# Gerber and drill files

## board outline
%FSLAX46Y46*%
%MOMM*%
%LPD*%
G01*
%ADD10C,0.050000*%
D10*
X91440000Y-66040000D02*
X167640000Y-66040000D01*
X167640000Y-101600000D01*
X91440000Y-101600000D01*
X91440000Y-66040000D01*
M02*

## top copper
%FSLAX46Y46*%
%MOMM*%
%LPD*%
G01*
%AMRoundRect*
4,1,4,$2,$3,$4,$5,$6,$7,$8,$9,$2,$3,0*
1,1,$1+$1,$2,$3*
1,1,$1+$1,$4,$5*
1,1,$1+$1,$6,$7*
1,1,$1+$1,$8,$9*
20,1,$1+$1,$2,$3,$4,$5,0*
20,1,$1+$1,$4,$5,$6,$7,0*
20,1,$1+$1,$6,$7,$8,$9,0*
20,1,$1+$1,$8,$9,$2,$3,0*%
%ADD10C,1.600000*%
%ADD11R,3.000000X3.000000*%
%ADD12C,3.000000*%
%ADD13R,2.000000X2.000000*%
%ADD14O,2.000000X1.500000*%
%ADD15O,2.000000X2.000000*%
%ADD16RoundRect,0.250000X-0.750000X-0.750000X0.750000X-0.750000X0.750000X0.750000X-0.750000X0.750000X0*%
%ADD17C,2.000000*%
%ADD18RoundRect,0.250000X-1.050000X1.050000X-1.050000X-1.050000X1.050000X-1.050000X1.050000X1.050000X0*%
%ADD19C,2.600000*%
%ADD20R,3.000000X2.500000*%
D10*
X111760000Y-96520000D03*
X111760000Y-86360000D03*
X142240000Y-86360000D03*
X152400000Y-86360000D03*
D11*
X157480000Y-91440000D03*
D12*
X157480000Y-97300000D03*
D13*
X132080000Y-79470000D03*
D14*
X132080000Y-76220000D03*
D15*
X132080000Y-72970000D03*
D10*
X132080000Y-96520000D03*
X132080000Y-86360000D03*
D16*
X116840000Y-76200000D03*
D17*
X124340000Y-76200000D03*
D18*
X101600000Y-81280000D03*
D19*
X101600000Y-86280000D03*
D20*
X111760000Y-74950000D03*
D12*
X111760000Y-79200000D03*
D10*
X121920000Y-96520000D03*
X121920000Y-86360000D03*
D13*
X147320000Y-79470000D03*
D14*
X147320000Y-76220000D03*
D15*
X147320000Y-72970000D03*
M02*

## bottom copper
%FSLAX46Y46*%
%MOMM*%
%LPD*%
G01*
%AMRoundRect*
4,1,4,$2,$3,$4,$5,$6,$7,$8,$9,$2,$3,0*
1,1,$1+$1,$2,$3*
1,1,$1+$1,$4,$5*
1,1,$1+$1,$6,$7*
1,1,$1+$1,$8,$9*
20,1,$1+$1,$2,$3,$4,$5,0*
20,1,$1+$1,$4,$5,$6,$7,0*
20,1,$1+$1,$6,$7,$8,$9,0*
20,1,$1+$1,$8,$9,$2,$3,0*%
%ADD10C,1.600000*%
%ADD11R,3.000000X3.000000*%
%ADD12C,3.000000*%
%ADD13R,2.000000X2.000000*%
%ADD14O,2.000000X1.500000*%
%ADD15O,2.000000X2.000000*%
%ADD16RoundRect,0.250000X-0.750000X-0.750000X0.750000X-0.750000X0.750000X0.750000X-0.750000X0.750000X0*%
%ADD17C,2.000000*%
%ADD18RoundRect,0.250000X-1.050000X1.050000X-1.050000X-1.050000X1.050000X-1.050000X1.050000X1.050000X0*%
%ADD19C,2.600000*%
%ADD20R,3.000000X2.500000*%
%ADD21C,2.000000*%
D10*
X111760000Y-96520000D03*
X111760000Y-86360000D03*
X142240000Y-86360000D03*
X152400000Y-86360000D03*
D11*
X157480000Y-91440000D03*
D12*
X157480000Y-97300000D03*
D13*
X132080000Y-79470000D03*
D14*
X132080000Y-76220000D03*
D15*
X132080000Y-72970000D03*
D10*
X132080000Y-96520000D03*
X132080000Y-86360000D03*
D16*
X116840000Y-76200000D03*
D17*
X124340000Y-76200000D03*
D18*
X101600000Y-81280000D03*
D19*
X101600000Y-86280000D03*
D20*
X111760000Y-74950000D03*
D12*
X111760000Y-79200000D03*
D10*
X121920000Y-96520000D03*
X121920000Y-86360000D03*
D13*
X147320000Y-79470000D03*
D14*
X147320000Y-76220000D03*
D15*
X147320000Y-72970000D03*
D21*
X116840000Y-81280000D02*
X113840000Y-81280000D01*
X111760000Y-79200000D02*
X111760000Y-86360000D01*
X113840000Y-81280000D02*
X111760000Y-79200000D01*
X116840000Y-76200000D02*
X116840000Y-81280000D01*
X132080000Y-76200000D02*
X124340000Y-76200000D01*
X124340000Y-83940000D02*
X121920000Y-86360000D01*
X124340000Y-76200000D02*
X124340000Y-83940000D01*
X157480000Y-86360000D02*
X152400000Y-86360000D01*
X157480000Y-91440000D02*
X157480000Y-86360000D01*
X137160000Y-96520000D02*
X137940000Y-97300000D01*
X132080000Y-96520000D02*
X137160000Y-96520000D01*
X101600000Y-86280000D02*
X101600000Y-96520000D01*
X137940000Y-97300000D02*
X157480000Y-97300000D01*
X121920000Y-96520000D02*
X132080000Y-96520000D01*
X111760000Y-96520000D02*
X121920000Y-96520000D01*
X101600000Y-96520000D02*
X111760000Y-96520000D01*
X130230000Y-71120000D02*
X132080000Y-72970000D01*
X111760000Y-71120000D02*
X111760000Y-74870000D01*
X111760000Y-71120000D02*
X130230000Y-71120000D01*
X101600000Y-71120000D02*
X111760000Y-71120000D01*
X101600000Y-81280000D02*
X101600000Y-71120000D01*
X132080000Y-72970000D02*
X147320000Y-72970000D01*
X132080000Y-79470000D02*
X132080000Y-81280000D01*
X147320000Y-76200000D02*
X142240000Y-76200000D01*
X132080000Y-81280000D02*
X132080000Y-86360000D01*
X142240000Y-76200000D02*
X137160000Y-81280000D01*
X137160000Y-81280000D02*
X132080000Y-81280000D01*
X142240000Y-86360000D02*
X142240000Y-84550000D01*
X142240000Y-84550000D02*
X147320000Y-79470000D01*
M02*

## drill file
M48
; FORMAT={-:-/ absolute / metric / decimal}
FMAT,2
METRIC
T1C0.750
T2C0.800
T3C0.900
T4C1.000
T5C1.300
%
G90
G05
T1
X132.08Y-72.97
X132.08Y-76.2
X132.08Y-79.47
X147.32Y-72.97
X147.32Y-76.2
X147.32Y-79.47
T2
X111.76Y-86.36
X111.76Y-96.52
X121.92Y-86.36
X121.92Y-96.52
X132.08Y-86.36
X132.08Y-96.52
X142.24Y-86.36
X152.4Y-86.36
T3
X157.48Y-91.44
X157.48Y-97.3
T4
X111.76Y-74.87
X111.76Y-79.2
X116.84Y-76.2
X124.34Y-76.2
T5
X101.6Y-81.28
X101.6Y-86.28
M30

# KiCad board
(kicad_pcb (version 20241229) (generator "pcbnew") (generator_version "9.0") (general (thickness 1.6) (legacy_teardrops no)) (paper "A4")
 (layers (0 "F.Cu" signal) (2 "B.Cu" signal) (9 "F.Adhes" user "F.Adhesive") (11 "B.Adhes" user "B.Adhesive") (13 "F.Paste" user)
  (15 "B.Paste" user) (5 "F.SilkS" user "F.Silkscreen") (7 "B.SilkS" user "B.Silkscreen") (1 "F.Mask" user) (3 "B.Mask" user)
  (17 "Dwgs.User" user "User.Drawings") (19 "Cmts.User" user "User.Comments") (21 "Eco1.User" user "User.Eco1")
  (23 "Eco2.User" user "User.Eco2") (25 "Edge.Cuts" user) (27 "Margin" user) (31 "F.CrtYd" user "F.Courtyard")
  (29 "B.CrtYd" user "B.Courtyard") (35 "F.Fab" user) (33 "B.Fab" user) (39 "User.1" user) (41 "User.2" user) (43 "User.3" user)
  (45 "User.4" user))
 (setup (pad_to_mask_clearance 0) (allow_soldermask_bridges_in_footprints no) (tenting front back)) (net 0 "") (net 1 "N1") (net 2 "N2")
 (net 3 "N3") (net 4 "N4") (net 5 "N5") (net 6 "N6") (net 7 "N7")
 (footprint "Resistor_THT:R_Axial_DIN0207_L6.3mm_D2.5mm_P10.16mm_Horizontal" (layer "F.Cu") (at 111.76 96.52 90)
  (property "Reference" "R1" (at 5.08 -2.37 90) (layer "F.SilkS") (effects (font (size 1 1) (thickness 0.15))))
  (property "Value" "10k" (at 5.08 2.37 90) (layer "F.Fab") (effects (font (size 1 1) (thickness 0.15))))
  (pad "1" thru_hole circle (at 0 0 90) (size 1.6 1.6) (drill 0.8) (layers "*.Cu" "*.Mask") (remove_unused_layers no) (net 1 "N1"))
  (pad "2" thru_hole circle (at 10.16 0 90) (size 1.6 1.6) (drill 0.8) (layers "*.Cu" "*.Mask") (remove_unused_layers no) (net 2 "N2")))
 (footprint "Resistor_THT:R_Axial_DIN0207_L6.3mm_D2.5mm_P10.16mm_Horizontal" (layer "F.Cu") (at 142.24 86.36)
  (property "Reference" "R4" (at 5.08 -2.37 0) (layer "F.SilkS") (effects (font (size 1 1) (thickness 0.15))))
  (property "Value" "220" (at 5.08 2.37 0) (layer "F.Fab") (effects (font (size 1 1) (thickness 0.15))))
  (pad "1" thru_hole circle (at 0 0) (size 1.6 1.6) (drill 0.8) (layers "*.Cu" "*.Mask") (remove_unused_layers no) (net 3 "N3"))
  (pad "2" thru_hole circle (at 10.16 0) (size 1.6 1.6) (drill 0.8) (layers "*.Cu" "*.Mask") (remove_unused_layers no) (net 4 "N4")))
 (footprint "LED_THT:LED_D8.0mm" (layer "F.Cu") (at 157.48 91.44 -90)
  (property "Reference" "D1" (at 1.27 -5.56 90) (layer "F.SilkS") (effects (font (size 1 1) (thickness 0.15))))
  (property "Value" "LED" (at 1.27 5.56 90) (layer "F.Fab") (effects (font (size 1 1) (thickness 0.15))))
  (pad "1" thru_hole rect (at 0 0 270) (size 3 3) (drill 0.9) (layers "*.Cu" "*.Mask") (remove_unused_layers no) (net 4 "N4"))
  (pad "2" thru_hole circle (at 5.86 0 270) (size 3 3) (drill 0.9) (layers "*.Cu" "*.Mask") (remove_unused_layers no) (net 1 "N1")))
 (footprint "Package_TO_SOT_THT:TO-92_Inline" (layer "F.Cu") (at 132.08 77.47 90)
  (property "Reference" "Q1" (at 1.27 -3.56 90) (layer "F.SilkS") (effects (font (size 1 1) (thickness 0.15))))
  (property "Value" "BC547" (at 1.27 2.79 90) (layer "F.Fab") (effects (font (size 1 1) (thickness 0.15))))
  (pad "1" thru_hole rect (at -2 0 90) (size 2 2) (drill 0.75) (layers "*.Cu" "*.Mask") (remove_unused_layers no) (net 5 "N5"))
  (pad "2" thru_hole oval (at 1.27 0 90) (size 1.5 2) (drill 0.75 (offset -0.02 0)) (layers "*.Cu" "*.Mask") (remove_unused_layers no)
   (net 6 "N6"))
  (pad "3" thru_hole oval (at 4.5 0 90) (size 2 2) (drill 0.75) (layers "*.Cu" "*.Mask") (remove_unused_layers no) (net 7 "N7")))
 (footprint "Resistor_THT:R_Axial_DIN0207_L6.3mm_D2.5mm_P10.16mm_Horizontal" (layer "F.Cu") (at 132.08 96.52 90)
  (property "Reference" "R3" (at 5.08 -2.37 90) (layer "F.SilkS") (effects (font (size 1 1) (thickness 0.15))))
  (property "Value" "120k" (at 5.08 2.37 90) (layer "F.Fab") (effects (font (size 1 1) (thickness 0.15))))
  (pad "1" thru_hole circle (at 0 0 90) (size 1.6 1.6) (drill 0.8) (layers "*.Cu" "*.Mask") (remove_unused_layers no) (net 1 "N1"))
  (pad "2" thru_hole circle (at 10.16 0 90) (size 1.6 1.6) (drill 0.8) (layers "*.Cu" "*.Mask") (remove_unused_layers no) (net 5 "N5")))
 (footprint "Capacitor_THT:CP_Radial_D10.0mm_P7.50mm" (layer "F.Cu") (at 116.84 76.2)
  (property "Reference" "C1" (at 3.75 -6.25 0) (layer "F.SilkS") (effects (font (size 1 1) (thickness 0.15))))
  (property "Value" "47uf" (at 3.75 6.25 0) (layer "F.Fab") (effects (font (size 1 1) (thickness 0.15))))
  (pad "1" thru_hole roundrect (at 0 0) (size 2 2) (drill 1) (layers "*.Cu" "*.Mask") (remove_unused_layers no) (roundrect_rratio 0.125)
   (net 2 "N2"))
  (pad "2" thru_hole circle (at 7.5 0) (size 2 2) (drill 1) (layers "*.Cu" "*.Mask") (remove_unused_layers no) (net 6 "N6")))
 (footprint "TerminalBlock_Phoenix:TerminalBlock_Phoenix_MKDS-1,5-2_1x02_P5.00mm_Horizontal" (layer "F.Cu") (at 101.6 81.28 -90)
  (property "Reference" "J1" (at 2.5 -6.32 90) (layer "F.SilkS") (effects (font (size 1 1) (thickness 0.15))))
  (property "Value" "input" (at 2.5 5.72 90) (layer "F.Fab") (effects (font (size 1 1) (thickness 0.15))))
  (pad "1" thru_hole roundrect (at 0 0 270) (size 2.6 2.6) (drill 1.3) (layers "*.Cu" "*.Mask") (remove_unused_layers no)
   (roundrect_rratio 0.096154) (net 7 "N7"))
  (pad "2" thru_hole circle (at 5 0 270) (size 2.6 2.6) (drill 1.3) (layers "*.Cu" "*.Mask") (remove_unused_layers no) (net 1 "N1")))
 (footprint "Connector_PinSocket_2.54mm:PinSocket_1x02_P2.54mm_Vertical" (layer "F.Cu") (at 111.76 76.2)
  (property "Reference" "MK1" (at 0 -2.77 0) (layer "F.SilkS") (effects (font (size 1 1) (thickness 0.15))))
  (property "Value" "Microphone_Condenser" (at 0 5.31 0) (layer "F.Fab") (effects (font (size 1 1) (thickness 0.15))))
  (pad "1" thru_hole rect (at 0 -1.33) (size 3 2.5) (drill 1 (offset 0 0.08)) (layers "*.Cu" "*.Mask") (remove_unused_layers no)
   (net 7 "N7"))
  (pad "2" thru_hole circle (at 0 3) (size 3 3) (drill 1) (layers "*.Cu" "*.Mask") (remove_unused_layers no) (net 2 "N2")))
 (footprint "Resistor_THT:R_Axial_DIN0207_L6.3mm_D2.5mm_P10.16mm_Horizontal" (layer "F.Cu") (at 121.92 96.52 90)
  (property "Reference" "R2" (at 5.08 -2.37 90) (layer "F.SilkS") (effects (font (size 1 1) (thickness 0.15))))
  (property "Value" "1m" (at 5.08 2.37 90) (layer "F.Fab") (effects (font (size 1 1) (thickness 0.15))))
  (pad "1" thru_hole circle (at 0 0 90) (size 1.6 1.6) (drill 0.8) (layers "*.Cu" "*.Mask") (remove_unused_layers no) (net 1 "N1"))
  (pad "2" thru_hole circle (at 10.16 0 90) (size 1.6 1.6) (drill 0.8) (layers "*.Cu" "*.Mask") (remove_unused_layers no) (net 6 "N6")))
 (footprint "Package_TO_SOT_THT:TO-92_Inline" (layer "F.Cu") (at 147.32 77.47 90)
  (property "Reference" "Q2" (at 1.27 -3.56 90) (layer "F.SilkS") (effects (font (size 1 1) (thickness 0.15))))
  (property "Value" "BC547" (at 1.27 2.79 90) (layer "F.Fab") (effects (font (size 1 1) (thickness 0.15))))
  (pad "1" thru_hole rect (at -2 0 90) (size 2 2) (drill 0.75) (layers "*.Cu" "*.Mask") (remove_unused_layers no) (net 3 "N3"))
  (pad "2" thru_hole oval (at 1.27 0 90) (size 1.5 2) (drill 0.75 (offset -0.02 0)) (layers "*.Cu" "*.Mask") (remove_unused_layers no)
   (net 5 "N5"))
  (pad "3" thru_hole oval (at 4.5 0 90) (size 2 2) (drill 0.75) (layers "*.Cu" "*.Mask") (remove_unused_layers no) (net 7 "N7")))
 (gr_rect (start 91.44 66.04) (end 167.64 101.6) (stroke (width 0.05) (type default)) (fill no) (layer "Edge.Cuts"))
 (segment (start 116.84 81.28) (end 113.84 81.28) (width 2) (layer "B.Cu") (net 2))
 (segment (start 111.76 79.2) (end 111.76 86.36) (width 2) (layer "B.Cu") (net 2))
 (segment (start 113.84 81.28) (end 111.76 79.2) (width 2) (layer "B.Cu") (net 2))
 (segment (start 116.84 76.2) (end 116.84 81.28) (width 2) (layer "B.Cu") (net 2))
 (segment (start 132.08 76.2) (end 124.34 76.2) (width 2) (layer "B.Cu") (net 6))
 (segment (start 124.34 83.94) (end 121.92 86.36) (width 2) (layer "B.Cu") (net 6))
 (segment (start 124.34 76.2) (end 124.34 83.94) (width 2) (layer "B.Cu") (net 6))
 (segment (start 157.48 86.36) (end 152.4 86.36) (width 2) (layer "B.Cu") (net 4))
 (segment (start 157.48 91.44) (end 157.48 86.36) (width 2) (layer "B.Cu") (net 4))
 (segment (start 137.16 96.52) (end 137.94 97.3) (width 2) (layer "B.Cu") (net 1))
 (segment (start 132.08 96.52) (end 137.16 96.52) (width 2) (layer "B.Cu") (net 1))
 (segment (start 101.6 86.28) (end 101.6 96.52) (width 2) (layer "B.Cu") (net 1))
 (segment (start 137.94 97.3) (end 157.48 97.3) (width 2) (layer "B.Cu") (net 1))
 (segment (start 121.92 96.52) (end 132.08 96.52) (width 2) (layer "B.Cu") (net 1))
 (segment (start 111.76 96.52) (end 121.92 96.52) (width 2) (layer "B.Cu") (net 1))
 (segment (start 101.6 96.52) (end 111.76 96.52) (width 2) (layer "B.Cu") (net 1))
 (segment (start 130.23 71.12) (end 132.08 72.97) (width 2) (layer "B.Cu") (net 7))
 (segment (start 111.76 71.12) (end 111.76 74.87) (width 2) (layer "B.Cu") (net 7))
 (segment (start 111.76 71.12) (end 130.23 71.12) (width 2) (layer "B.Cu") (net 7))
 (segment (start 101.6 71.12) (end 111.76 71.12) (width 2) (layer "B.Cu") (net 7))
 (segment (start 101.6 81.28) (end 101.6 71.12) (width 2) (layer "B.Cu") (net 7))
 (segment (start 132.08 72.97) (end 147.32 72.97) (width 2) (layer "B.Cu") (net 7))
 (segment (start 132.08 79.47) (end 132.08 81.28) (width 2) (layer "B.Cu") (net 5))
 (segment (start 147.32 76.2) (end 142.24 76.2) (width 2) (layer "B.Cu") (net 5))
 (segment (start 132.08 81.28) (end 132.08 86.36) (width 2) (layer "B.Cu") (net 5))
 (segment (start 142.24 76.2) (end 137.16 81.28) (width 2) (layer "B.Cu") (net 5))
 (segment (start 137.16 81.28) (end 132.08 81.28) (width 2) (layer "B.Cu") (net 5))
 (segment (start 142.24 86.36) (end 142.24 84.55) (width 2) (layer "B.Cu") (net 3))
 (segment (start 142.24 84.55) (end 147.32 79.47) (width 2) (layer "B.Cu") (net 3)))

